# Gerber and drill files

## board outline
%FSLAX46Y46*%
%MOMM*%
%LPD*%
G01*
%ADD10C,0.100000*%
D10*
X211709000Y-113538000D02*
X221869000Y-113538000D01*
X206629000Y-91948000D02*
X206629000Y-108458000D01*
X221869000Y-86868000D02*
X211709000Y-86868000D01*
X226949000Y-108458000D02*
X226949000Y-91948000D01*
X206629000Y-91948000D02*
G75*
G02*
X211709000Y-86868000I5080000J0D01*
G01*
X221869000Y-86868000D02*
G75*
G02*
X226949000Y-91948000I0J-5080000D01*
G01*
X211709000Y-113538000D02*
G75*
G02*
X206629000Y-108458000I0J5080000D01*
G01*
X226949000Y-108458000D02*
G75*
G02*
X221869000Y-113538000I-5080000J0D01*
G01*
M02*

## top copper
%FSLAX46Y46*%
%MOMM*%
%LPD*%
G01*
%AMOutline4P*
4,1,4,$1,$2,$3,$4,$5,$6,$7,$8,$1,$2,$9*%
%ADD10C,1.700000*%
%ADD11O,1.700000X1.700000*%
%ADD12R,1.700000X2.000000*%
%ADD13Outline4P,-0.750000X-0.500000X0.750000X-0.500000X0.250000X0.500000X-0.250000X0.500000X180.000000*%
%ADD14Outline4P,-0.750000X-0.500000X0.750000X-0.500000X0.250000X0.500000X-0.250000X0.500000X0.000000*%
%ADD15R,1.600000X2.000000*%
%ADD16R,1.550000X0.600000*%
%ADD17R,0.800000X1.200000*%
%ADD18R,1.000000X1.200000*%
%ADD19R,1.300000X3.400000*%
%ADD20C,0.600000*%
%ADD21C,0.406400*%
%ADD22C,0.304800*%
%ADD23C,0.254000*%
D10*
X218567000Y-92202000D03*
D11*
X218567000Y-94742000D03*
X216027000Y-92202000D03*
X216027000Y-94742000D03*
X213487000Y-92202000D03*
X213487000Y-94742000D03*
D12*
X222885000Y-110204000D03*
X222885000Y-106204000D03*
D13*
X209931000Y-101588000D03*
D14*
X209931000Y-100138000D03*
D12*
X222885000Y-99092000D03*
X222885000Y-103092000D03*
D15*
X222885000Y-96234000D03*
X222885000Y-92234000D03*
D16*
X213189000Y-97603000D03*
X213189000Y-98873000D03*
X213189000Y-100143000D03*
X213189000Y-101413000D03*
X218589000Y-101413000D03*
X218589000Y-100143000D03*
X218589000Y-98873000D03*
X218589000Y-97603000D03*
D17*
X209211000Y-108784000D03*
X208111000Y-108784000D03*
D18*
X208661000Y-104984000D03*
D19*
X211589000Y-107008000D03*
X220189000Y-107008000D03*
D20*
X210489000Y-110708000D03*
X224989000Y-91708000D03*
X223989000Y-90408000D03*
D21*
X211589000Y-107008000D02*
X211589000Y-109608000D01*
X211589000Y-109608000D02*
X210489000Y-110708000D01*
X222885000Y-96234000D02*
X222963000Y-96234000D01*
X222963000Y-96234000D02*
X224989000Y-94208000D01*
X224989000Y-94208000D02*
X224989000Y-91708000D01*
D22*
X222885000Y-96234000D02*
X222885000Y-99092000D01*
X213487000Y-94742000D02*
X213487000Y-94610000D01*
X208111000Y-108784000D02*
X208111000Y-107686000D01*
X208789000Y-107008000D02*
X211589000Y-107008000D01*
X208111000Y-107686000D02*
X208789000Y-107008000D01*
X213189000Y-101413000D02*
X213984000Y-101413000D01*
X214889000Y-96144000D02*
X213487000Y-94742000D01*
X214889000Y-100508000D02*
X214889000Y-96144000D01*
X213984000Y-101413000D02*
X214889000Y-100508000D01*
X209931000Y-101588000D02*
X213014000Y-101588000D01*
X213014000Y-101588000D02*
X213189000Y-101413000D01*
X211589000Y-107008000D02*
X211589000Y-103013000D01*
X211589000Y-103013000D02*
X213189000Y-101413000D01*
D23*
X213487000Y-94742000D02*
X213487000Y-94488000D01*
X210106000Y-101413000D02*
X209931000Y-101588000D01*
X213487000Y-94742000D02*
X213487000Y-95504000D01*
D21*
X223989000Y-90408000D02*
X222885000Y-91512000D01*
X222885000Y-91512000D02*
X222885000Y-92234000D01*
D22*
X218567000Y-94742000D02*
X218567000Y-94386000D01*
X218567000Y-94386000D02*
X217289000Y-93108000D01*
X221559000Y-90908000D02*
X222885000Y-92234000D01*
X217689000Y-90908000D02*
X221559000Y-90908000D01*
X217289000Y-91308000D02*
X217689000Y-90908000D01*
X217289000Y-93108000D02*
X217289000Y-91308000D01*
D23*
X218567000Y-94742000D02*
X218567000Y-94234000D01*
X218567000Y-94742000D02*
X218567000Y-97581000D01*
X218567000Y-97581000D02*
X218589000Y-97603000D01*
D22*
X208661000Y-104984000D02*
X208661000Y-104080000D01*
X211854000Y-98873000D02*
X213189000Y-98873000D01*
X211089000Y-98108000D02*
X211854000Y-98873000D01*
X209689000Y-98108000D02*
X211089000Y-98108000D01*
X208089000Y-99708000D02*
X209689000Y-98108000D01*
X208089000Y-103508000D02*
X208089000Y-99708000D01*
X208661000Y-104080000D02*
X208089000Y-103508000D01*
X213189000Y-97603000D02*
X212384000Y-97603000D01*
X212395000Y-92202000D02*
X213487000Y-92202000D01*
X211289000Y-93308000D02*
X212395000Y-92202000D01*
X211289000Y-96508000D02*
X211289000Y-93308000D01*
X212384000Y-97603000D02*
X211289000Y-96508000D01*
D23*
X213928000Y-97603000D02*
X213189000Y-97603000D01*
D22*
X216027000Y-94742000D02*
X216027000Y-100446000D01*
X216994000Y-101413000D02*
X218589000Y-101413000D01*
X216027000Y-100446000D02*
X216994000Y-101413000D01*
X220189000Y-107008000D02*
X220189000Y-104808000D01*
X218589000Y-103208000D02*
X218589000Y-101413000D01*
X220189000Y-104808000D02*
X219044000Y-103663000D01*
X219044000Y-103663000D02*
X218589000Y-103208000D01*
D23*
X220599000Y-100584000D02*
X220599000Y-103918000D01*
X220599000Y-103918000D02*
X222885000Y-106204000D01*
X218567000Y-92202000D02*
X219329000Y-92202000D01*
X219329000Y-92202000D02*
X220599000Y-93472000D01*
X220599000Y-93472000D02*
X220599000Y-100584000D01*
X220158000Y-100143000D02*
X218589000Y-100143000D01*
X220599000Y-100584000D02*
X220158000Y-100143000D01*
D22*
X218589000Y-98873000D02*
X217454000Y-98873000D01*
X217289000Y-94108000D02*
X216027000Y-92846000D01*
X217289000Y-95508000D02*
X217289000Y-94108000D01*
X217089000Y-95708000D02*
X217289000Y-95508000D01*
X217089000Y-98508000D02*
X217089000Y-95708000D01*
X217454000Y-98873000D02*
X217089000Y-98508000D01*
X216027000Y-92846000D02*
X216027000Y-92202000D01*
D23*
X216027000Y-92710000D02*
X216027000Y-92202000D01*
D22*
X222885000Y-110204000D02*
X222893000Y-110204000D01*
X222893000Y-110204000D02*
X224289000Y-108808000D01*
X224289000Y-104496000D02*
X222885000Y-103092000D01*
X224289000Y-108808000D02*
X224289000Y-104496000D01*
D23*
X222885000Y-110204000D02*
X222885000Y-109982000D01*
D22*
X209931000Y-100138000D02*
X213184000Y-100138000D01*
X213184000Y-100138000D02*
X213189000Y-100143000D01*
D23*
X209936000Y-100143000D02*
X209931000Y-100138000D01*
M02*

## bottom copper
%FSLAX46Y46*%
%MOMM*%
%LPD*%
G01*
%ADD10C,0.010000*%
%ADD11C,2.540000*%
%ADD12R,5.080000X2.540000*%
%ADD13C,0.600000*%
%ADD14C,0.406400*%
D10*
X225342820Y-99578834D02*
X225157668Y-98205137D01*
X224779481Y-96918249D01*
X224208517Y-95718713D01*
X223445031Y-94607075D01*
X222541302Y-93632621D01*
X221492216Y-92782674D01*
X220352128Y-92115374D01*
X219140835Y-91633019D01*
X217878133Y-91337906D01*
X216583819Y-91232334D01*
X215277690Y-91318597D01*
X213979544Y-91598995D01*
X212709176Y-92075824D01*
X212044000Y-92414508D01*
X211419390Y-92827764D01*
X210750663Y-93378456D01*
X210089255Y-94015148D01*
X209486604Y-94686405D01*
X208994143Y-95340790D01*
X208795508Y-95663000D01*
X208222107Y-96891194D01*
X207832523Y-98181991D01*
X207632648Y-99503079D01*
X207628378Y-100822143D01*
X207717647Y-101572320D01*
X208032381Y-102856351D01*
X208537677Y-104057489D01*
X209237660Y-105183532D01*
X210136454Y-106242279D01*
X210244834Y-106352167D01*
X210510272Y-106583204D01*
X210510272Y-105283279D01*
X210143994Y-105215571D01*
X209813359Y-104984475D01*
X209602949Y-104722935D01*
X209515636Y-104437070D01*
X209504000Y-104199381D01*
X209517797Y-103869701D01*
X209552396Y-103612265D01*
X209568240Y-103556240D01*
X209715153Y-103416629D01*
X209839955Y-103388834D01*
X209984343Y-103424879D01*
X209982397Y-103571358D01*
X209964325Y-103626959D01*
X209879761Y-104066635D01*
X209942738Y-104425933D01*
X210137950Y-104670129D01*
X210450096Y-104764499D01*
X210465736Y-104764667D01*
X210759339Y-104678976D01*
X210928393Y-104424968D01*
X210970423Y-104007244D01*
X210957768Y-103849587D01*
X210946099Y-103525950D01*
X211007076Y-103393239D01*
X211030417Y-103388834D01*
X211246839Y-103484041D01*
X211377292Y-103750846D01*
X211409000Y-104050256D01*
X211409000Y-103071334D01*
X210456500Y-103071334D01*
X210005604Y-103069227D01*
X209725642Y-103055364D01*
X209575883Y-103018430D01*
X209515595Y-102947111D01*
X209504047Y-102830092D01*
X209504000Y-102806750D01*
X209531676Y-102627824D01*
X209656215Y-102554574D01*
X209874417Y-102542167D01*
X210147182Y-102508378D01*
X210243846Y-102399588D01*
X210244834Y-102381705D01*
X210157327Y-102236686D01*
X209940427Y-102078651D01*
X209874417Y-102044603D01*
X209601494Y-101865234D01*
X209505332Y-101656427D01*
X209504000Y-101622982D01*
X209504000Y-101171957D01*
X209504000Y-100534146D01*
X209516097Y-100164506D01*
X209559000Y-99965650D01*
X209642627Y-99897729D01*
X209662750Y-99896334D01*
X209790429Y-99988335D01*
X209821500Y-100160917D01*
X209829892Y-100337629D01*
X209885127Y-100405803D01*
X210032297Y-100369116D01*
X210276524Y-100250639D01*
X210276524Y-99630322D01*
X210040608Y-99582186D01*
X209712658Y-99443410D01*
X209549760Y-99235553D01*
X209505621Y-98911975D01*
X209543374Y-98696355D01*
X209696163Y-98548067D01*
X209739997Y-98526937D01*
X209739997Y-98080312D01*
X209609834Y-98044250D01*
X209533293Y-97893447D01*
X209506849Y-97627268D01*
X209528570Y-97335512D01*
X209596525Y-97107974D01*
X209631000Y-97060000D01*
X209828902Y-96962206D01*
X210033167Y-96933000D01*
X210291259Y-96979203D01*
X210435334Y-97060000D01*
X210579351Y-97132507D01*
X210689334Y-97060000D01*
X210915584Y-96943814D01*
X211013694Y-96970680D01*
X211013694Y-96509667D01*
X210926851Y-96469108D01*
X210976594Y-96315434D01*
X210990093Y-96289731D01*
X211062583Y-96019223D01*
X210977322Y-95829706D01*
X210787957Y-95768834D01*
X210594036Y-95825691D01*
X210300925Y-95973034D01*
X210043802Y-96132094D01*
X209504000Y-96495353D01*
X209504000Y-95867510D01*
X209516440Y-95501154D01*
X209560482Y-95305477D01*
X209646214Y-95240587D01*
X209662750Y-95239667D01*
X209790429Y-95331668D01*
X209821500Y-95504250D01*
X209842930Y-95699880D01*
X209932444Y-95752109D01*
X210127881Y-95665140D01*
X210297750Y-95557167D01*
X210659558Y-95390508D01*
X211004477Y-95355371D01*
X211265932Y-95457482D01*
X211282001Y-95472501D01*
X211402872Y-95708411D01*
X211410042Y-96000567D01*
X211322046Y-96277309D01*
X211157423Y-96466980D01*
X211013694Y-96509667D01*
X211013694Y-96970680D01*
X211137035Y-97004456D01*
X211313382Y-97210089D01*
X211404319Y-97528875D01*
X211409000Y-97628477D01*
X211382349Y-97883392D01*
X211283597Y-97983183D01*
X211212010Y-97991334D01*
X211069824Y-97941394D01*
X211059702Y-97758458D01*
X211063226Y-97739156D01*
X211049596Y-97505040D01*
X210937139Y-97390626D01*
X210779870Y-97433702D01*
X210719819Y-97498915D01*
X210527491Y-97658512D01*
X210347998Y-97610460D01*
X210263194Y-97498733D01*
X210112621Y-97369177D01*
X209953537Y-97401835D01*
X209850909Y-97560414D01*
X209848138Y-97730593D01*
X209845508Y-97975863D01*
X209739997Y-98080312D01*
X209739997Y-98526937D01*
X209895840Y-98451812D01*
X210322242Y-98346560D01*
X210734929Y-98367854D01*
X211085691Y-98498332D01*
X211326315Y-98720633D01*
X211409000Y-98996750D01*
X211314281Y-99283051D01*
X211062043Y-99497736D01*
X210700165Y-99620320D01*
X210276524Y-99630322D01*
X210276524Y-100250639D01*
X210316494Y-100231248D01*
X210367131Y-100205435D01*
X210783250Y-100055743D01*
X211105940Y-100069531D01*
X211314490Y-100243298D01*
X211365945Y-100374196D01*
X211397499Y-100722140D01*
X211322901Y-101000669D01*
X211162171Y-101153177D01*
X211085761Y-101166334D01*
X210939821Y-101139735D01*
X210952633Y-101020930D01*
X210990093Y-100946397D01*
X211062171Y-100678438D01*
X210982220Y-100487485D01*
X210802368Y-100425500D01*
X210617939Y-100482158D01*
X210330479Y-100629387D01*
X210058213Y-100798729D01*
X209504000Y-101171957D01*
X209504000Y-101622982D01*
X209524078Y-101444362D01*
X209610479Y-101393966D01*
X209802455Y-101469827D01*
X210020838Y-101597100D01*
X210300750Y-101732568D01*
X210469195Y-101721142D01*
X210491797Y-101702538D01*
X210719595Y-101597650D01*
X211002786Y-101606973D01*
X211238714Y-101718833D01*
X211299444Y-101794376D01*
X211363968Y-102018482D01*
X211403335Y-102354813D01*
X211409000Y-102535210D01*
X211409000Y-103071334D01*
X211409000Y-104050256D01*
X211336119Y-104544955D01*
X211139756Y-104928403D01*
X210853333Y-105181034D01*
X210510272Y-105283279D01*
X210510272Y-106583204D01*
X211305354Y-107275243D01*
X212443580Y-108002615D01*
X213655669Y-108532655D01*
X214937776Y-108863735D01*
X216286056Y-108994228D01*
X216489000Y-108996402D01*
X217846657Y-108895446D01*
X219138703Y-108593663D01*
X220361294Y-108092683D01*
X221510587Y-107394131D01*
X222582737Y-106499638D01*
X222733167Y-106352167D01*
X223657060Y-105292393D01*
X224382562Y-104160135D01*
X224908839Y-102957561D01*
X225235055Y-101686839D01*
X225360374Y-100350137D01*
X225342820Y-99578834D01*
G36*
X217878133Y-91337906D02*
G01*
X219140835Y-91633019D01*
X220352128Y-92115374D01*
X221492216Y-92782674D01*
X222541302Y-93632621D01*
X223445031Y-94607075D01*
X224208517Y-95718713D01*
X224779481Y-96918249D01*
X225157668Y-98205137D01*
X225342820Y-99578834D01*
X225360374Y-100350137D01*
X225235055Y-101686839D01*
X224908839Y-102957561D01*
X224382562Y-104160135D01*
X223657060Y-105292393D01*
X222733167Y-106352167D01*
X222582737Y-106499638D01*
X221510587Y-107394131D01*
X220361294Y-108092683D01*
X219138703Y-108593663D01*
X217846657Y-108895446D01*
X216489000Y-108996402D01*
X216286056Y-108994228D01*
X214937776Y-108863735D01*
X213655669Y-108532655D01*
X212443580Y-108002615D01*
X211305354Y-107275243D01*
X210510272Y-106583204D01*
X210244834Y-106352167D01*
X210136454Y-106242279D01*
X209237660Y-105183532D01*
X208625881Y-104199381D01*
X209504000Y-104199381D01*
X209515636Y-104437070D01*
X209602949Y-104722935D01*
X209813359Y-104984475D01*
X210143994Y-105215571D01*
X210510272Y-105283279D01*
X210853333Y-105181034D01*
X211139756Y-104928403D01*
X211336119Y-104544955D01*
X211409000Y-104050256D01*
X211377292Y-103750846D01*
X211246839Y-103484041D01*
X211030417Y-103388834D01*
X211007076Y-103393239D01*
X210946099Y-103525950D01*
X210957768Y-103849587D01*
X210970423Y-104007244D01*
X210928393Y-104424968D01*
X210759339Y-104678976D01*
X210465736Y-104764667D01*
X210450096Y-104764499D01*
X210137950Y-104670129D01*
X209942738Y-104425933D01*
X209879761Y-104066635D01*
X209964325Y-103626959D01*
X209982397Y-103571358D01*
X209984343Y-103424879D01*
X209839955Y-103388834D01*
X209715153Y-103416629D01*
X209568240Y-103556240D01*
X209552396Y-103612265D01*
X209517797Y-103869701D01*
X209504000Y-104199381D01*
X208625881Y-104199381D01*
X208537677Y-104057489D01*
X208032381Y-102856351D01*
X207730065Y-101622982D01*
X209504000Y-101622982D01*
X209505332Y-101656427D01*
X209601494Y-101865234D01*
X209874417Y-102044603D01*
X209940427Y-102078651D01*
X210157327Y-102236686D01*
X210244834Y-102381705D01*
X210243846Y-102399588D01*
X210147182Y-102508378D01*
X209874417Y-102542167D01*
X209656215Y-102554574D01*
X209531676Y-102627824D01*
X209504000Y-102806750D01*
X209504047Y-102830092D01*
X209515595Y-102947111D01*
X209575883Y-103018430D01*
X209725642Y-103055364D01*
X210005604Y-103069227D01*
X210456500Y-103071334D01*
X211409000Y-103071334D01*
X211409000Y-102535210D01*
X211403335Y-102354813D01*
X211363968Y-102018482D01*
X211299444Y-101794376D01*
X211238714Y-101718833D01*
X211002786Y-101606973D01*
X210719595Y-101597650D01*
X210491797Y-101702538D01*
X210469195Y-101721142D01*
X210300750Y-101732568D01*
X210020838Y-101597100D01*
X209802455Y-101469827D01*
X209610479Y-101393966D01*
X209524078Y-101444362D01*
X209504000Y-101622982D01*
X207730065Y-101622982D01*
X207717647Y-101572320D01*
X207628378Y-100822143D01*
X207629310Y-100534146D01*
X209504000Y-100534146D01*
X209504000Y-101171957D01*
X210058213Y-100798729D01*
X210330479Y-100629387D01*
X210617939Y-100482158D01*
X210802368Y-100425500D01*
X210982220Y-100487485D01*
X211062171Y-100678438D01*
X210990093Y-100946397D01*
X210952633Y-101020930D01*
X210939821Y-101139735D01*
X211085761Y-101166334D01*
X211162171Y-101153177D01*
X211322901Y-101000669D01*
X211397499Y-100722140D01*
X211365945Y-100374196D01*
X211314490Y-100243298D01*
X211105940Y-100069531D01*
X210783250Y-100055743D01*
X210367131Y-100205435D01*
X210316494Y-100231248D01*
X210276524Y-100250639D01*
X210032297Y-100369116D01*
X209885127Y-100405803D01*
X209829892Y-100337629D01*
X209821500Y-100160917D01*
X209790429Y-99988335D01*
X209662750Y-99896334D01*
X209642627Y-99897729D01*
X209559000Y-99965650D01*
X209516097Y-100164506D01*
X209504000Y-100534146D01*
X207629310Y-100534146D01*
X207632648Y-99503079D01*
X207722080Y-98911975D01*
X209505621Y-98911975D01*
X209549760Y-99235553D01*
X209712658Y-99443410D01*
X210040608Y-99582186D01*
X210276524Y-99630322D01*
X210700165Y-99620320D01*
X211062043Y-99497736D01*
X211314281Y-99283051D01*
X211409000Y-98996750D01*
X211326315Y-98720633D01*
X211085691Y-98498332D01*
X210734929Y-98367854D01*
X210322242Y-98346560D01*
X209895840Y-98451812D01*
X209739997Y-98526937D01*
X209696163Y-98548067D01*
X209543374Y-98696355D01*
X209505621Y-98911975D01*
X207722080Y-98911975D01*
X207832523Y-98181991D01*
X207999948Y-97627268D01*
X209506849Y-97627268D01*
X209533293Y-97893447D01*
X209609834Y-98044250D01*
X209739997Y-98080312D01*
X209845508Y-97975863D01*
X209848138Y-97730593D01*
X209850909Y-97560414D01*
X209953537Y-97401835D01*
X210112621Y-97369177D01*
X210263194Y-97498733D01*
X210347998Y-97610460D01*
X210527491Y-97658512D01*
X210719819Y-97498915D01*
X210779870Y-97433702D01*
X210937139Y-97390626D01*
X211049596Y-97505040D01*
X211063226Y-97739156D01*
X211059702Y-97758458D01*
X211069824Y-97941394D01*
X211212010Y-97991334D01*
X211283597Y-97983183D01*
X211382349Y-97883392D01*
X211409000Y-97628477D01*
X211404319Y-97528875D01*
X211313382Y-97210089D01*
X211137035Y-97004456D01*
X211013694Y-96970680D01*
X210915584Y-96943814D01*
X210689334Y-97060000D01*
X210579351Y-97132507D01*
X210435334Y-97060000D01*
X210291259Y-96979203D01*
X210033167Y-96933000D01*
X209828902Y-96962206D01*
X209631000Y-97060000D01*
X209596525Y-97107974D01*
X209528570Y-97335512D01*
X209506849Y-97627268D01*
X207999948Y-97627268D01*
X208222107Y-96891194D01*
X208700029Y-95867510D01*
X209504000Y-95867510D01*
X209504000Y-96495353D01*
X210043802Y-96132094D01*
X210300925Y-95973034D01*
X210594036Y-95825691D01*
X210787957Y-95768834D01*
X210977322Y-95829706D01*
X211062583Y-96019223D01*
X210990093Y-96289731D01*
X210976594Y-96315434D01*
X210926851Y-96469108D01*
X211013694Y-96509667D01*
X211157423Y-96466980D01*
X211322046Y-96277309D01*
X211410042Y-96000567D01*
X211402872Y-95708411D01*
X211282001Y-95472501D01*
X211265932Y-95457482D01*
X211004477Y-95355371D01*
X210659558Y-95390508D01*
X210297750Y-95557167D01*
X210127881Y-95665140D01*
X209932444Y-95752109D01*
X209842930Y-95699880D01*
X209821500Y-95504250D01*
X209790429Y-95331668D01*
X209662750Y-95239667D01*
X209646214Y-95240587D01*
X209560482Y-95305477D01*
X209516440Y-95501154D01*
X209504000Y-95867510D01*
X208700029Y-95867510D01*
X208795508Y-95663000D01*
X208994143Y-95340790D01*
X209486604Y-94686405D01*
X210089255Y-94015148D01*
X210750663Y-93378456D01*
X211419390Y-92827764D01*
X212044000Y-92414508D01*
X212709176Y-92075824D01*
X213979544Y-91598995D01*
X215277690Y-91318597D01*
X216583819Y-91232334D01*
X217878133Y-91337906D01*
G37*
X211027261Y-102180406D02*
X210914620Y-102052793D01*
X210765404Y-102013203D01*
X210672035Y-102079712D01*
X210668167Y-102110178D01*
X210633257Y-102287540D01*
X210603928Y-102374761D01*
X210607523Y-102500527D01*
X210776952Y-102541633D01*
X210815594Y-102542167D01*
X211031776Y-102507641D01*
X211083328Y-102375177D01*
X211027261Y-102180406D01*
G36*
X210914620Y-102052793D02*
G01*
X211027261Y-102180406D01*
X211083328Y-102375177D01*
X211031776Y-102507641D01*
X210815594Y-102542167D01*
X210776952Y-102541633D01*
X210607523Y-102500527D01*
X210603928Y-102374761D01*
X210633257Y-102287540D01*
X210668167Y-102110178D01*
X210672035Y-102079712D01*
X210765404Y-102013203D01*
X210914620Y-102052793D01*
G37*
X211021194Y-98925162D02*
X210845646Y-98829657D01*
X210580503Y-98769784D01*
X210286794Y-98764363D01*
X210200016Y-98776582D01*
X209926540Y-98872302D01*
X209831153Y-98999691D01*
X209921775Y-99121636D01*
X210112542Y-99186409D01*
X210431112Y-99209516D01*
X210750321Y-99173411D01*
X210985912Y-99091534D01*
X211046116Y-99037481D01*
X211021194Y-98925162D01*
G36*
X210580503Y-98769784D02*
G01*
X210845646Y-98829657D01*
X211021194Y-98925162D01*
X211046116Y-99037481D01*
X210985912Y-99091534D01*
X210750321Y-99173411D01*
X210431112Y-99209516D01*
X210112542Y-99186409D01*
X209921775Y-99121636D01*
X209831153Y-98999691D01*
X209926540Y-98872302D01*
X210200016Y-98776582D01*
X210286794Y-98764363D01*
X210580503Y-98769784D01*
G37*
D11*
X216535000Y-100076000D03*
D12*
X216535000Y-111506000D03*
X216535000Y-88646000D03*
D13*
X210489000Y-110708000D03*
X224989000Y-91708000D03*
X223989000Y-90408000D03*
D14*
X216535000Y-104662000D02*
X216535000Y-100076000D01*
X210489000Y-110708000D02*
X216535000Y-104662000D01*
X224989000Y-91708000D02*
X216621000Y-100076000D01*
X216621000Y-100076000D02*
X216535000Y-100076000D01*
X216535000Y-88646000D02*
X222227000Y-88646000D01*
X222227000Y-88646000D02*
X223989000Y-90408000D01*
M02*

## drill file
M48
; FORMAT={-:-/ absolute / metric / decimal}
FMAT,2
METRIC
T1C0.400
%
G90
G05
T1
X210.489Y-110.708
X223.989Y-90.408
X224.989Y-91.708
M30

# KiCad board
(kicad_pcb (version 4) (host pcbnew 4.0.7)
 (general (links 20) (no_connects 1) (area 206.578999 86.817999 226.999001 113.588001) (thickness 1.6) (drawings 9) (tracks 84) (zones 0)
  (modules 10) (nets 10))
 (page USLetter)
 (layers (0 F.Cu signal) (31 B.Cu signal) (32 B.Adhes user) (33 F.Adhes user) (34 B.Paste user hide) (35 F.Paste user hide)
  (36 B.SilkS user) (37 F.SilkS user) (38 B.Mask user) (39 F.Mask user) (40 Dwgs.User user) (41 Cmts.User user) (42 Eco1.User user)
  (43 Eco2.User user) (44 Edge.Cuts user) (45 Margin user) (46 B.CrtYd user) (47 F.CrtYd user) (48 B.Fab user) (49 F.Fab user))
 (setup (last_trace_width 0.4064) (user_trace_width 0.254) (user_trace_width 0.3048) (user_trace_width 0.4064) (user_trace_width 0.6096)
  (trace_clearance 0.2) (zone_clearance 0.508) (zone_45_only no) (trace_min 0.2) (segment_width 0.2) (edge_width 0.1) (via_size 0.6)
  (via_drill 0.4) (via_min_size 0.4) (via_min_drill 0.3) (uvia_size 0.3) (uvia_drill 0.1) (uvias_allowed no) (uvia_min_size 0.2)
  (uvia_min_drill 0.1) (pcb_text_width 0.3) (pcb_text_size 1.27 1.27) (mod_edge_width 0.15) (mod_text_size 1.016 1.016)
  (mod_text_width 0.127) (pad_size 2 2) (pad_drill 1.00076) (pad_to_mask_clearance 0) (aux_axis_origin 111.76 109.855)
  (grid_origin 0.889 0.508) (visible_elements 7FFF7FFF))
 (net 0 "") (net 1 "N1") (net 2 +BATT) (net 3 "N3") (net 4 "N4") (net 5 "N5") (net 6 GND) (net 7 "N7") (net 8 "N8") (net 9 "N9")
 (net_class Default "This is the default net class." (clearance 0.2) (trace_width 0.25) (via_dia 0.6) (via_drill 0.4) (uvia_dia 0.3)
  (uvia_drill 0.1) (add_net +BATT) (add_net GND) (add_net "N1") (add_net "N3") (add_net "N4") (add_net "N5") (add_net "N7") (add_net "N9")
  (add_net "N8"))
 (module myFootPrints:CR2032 (layer B.Cu) (at 216.489 100.108 90)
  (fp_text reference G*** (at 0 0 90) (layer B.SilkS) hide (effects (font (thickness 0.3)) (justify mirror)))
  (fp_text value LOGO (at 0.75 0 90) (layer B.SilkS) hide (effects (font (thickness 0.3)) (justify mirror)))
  (fp_poly
   (pts (xy 0.529166 8.85382) (xy 1.902863 8.668668) (xy 3.189751 8.290481) (xy 4.389287 7.719517) (xy 5.500925 6.956031)
    (xy 6.475379 6.052302) (xy 7.325326 5.003216) (xy 7.992626 3.863128) (xy 8.474981 2.651835) (xy 8.770094 1.389133)
    (xy 8.875666 0.094819) (xy 8.789403 -1.21131) (xy 8.509005 -2.509456) (xy 8.032176 -3.779824) (xy 7.693492 -4.445)
    (xy 7.280236 -5.06961) (xy 6.729544 -5.738337) (xy 6.092852 -6.399745) (xy 5.421595 -7.002396) (xy 4.76721 -7.494857)
    (xy 4.445 -7.693492) (xy 3.216806 -8.266893) (xy 1.926009 -8.656477) (xy 0.604921 -8.856352) (xy -0.714143 -8.860622)
    (xy -1.46432 -8.771353) (xy -2.748351 -8.456619) (xy -3.949489 -7.951323) (xy -5.075532 -7.25134) (xy -6.134279 -6.352546)
    (xy -6.244167 -6.244166) (xy -6.475204 -5.978728) (xy -5.175279 -5.978728) (xy -5.107571 -6.345006) (xy -4.876475 -6.675641)
    (xy -4.614935 -6.886051) (xy -4.32907 -6.973364) (xy -4.091381 -6.985) (xy -3.761701 -6.971203) (xy -3.504265 -6.936604)
    (xy -3.44824 -6.92076) (xy -3.308629 -6.773847) (xy -3.280834 -6.649045) (xy -3.316879 -6.504657) (xy -3.463358 -6.506603)
    (xy -3.518959 -6.524675) (xy -3.958635 -6.609239) (xy -4.317933 -6.546262) (xy -4.562129 -6.35105) (xy -4.656499 -6.038904)
    (xy -4.656667 -6.023264) (xy -4.570976 -5.729661) (xy -4.316968 -5.560607) (xy -3.899244 -5.518577) (xy -3.741587 -5.531232)
    (xy -3.41795 -5.542901) (xy -3.285239 -5.481924) (xy -3.280834 -5.458583) (xy -3.376041 -5.242161) (xy -3.642846 -5.111708)
    (xy -3.942256 -5.08) (xy -2.963334 -5.08) (xy -2.963334 -6.0325) (xy -2.961227 -6.483396) (xy -2.947364 -6.763358)
    (xy -2.91043 -6.913117) (xy -2.839111 -6.973405) (xy -2.722092 -6.984953) (xy -2.69875 -6.985) (xy -2.519824 -6.957324)
    (xy -2.446574 -6.832785) (xy -2.434167 -6.614583) (xy -2.400378 -6.341818) (xy -2.291588 -6.245154) (xy -2.273705 -6.244166)
    (xy -2.128686 -6.331673) (xy -1.970651 -6.548573) (xy -1.936603 -6.614583) (xy -1.757234 -6.887506) (xy -1.548427 -6.983668)
    (xy -1.514982 -6.985) (xy -1.063957 -6.985) (xy -0.426146 -6.985) (xy -0.056506 -6.972903) (xy 0.14235 -6.93) (xy 0.210271 -6.846373)
    (xy 0.211666 -6.82625) (xy 0.119665 -6.698571) (xy -0.052917 -6.6675) (xy -0.229629 -6.659108) (xy -0.297803 -6.603873)
    (xy -0.261116 -6.456703) (xy -0.142639 -6.212476) (xy 0.477678 -6.212476) (xy 0.525814 -6.448392) (xy 0.66459 -6.776342)
    (xy 0.872447 -6.93924) (xy 1.196025 -6.983379) (xy 1.411645 -6.945626) (xy 1.559933 -6.792837) (xy 1.581063 -6.749003)
    (xy 2.027688 -6.749003) (xy 2.06375 -6.879166) (xy 2.214553 -6.955707) (xy 2.480732 -6.982151) (xy 2.772488 -6.96043)
    (xy 3.000026 -6.892475) (xy 3.048 -6.858) (xy 3.145794 -6.660098) (xy 3.175 -6.455833) (xy 3.128797 -6.197741) (xy 3.048 -6.053666)
    (xy 2.975493 -5.909649) (xy 3.048 -5.799666) (xy 3.164186 -5.573416) (xy 3.13732 -5.475306) (xy 3.598333 -5.475306)
    (xy 3.638892 -5.562149) (xy 3.792566 -5.512406) (xy 3.818269 -5.498907) (xy 4.088777 -5.426417) (xy 4.278294 -5.511678)
    (xy 4.339166 -5.701043) (xy 4.282309 -5.894964) (xy 4.134966 -6.188075) (xy 3.975906 -6.445198) (xy 3.612647 -6.985) (xy 4.24049 -6.985)
    (xy 4.606846 -6.97256) (xy 4.802523 -6.928518) (xy 4.867413 -6.842786) (xy 4.868333 -6.82625) (xy 4.776332 -6.698571)
    (xy 4.60375 -6.6675) (xy 4.40812 -6.64607) (xy 4.355891 -6.556556) (xy 4.44286 -6.361119) (xy 4.550833 -6.19125) (xy 4.717492 -5.829442)
    (xy 4.752629 -5.484523) (xy 4.650518 -5.223068) (xy 4.635499 -5.206999) (xy 4.399589 -5.086128) (xy 4.107433 -5.078958)
    (xy 3.830691 -5.166954) (xy 3.64102 -5.331577) (xy 3.598333 -5.475306) (xy 3.13732 -5.475306) (xy 3.103544 -5.351965)
    (xy 2.897911 -5.175618) (xy 2.579125 -5.084681) (xy 2.479523 -5.08) (xy 2.224608 -5.106651) (xy 2.124817 -5.205403)
    (xy 2.116666 -5.27699) (xy 2.166606 -5.419176) (xy 2.349542 -5.429298) (xy 2.368844 -5.425774) (xy 2.60296 -5.439404)
    (xy 2.717374 -5.551861) (xy 2.674298 -5.70913) (xy 2.609085 -5.769181) (xy 2.449488 -5.961509) (xy 2.49754 -6.141002)
    (xy 2.609267 -6.225806) (xy 2.738823 -6.376379) (xy 2.706165 -6.535463) (xy 2.547586 -6.638091) (xy 2.377407 -6.640862)
    (xy 2.132137 -6.643492) (xy 2.027688 -6.749003) (xy 1.581063 -6.749003) (xy 1.656188 -6.59316) (xy 1.76144 -6.166758)
    (xy 1.740146 -5.754071) (xy 1.609668 -5.403309) (xy 1.387367 -5.162685) (xy 1.11125 -5.08) (xy 0.824949 -5.174719)
    (xy 0.610264 -5.426957) (xy 0.48768 -5.788835) (xy 0.477678 -6.212476) (xy -0.142639 -6.212476) (xy -0.123248 -6.172506)
    (xy -0.097435 -6.121869) (xy 0.052257 -5.70575) (xy 0.038469 -5.38306) (xy -0.135298 -5.17451) (xy -0.266196 -5.123055)
    (xy -0.61414 -5.091501) (xy -0.892669 -5.166099) (xy -1.045177 -5.326829) (xy -1.058334 -5.403239) (xy -1.031735 -5.549179)
    (xy -0.91293 -5.536367) (xy -0.838397 -5.498907) (xy -0.570438 -5.426829) (xy -0.379485 -5.50678) (xy -0.3175 -5.686632)
    (xy -0.374158 -5.871061) (xy -0.521387 -6.158521) (xy -0.690729 -6.430787) (xy -1.063957 -6.985) (xy -1.514982 -6.985)
    (xy -1.336362 -6.964922) (xy -1.285966 -6.878521) (xy -1.361827 -6.686545) (xy -1.4891 -6.468162) (xy -1.624568 -6.18825)
    (xy -1.613142 -6.019805) (xy -1.594538 -5.997203) (xy -1.48965 -5.769405) (xy -1.498973 -5.486214) (xy -1.610833 -5.250286)
    (xy -1.686376 -5.189556) (xy -1.910482 -5.125032) (xy -2.246813 -5.085665) (xy -2.42721 -5.08) (xy -2.963334 -5.08) (xy -3.942256 -5.08)
    (xy -4.436955 -5.152881) (xy -4.820403 -5.349244) (xy -5.073034 -5.635667) (xy -5.175279 -5.978728) (xy -6.475204 -5.978728)
    (xy -7.167243 -5.183646) (xy -7.894615 -4.04542) (xy -8.424655 -2.833331) (xy -8.755735 -1.551224) (xy -8.886228 -0.202944)
    (xy -8.888402 0) (xy -8.787446 1.357657) (xy -8.485663 2.649703) (xy -7.984683 3.872294) (xy -7.286131 5.021587) (xy -6.391638 6.093737)
    (xy -6.244167 6.244167) (xy -5.184393 7.16806) (xy -4.052135 7.893562) (xy -2.849561 8.419839) (xy -1.578839 8.746055)
    (xy -0.242137 8.871374) (xy 0.529166 8.85382))
   (layer B.Cu) (width 0.01))
  (fp_poly
   (pts (xy -2.072406 -5.461739) (xy -1.944793 -5.57438) (xy -1.905203 -5.723596) (xy -1.971712 -5.816965) (xy -2.002178 -5.820833)
    (xy -2.17954 -5.855743) (xy -2.266761 -5.885072) (xy -2.392527 -5.881477) (xy -2.433633 -5.712048) (xy -2.434167 -5.673406)
    (xy -2.399641 -5.457224) (xy -2.267177 -5.405672) (xy -2.072406 -5.461739))
   (layer B.Cu) (width 0.01))
  (fp_poly
   (pts (xy 1.182838 -5.467806) (xy 1.278343 -5.643354) (xy 1.338216 -5.908497) (xy 1.343637 -6.202206) (xy 1.331418 -6.288984)
    (xy 1.235698 -6.56246) (xy 1.108309 -6.657847) (xy 0.986364 -6.567225) (xy 0.921591 -6.376458) (xy 0.898484 -6.057888)
    (xy 0.934589 -5.738679) (xy 1.016466 -5.503088) (xy 1.070519 -5.442884) (xy 1.182838 -5.467806))
   (layer B.Cu) (width 0.01))
  (pad 3 smd circle (at 0 0 90) (size 17.78 17.78) (layers B.Paste B.Mask)))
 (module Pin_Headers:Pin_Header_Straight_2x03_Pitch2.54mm (layer F.Cu) (at 218.567 92.202 270)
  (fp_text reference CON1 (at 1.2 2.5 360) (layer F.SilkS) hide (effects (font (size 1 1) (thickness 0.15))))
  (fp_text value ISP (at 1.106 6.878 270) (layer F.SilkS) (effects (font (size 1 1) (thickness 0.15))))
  (pad 1 smd circle (at 0 0 270) (size 1.7 1.7) (layers F.Cu F.Paste F.Mask) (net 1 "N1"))
  (pad 2 smd oval (at 2.54 0 270) (size 1.7 1.7) (layers F.Cu F.Paste F.Mask) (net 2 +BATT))
  (pad 3 smd oval (at 0 2.54 270) (size 1.7 1.7) (layers F.Cu F.Paste F.Mask) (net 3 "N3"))
  (pad 4 smd oval (at 2.54 2.54 270) (size 1.7 1.7) (layers F.Cu F.Paste F.Mask) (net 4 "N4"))
  (pad 5 smd oval (at 0 5.08 270) (size 1.7 1.7) (layers F.Cu F.Paste F.Mask) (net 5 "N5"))
  (pad 6 smd oval (at 2.54 5.08 270) (size 1.7 1.7) (layers F.Cu F.Paste F.Mask) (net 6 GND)))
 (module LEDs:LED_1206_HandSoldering (layer F.Cu) (at 222.885 108.204 90)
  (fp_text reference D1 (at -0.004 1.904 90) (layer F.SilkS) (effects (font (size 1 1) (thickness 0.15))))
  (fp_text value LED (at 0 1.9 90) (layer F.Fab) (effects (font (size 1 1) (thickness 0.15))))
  (pad 1 smd rect (at -2 0 90) (size 2 1.7) (layers F.Cu F.Paste F.Mask) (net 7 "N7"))
  (pad 2 smd rect (at 2 0 90) (size 2 1.7) (layers F.Cu F.Paste F.Mask) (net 1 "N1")))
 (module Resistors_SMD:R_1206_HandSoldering (layer F.Cu) (at 209.931 100.838 90)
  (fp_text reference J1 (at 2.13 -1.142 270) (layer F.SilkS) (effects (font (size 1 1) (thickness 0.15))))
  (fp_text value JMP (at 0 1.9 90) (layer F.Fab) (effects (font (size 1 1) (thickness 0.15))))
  (pad 1 smd trapezoid (at -0.75 0 180) (size 1 1) (rect_delta 0 0.5) (layers F.Cu F.Paste F.Mask) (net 6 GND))
  (pad 2 smd trapezoid (at 0.7 0) (size 1 1) (rect_delta 0 0.5) (layers F.Cu F.Paste F.Mask) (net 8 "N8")))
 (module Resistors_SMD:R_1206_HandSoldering (layer F.Cu) (at 222.885 101.092 270)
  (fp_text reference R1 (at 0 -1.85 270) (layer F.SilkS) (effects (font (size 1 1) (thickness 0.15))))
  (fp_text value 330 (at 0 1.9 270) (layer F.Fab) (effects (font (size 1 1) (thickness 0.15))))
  (pad 1 smd rect (at -2 0 270) (size 2 1.7) (layers F.Cu F.Paste F.Mask) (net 6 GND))
  (pad 2 smd rect (at 2 0 270) (size 2 1.7) (layers F.Cu F.Paste F.Mask) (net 7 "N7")))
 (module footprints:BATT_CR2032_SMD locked (layer B.Cu) (at 216.535 100.076 90)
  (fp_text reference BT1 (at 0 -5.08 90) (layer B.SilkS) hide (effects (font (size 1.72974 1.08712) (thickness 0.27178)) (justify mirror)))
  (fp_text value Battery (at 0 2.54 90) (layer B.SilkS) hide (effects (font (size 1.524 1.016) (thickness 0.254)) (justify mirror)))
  (pad 2 smd circle (at 0 0 90) (size 2.54 2.54) (layers B.Cu B.Paste B.Mask) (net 6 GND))
  (pad 1 smd rect (at -11.43 0 90) (size 2.54 5.08) (layers B.Cu B.Paste B.Mask) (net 2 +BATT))
  (pad 1 smd rect (at 11.43 0 90) (size 2.54 5.08) (layers B.Cu B.Paste B.Mask) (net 2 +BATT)))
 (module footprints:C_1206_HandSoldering (layer F.Cu) (at 222.885 94.234 90)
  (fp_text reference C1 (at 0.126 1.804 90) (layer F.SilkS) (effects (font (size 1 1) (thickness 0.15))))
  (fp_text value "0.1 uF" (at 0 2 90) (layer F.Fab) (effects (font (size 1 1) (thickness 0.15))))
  (pad 1 smd rect (at -2 0 90) (size 2 1.6) (layers F.Cu F.Paste F.Mask) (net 6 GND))
  (pad 2 smd rect (at 2 0 90) (size 2 1.6) (layers F.Cu F.Paste F.Mask) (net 2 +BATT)))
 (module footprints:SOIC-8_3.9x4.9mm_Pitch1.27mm (layer F.Cu) (at 215.889 99.508)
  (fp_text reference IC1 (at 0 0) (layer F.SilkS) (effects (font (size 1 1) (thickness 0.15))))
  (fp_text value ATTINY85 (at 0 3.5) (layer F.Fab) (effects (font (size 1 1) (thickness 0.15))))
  (pad 1 smd rect (at -2.7 -1.905) (size 1.55 0.6) (layers F.Cu F.Paste F.Mask) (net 5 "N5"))
  (pad 2 smd rect (at -2.7 -0.635) (size 1.55 0.6) (layers F.Cu F.Paste F.Mask) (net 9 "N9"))
  (pad 3 smd rect (at -2.7 0.635) (size 1.55 0.6) (layers F.Cu F.Paste F.Mask) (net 8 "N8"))
  (pad 4 smd rect (at -2.7 1.905) (size 1.55 0.6) (layers F.Cu F.Paste F.Mask) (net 6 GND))
  (pad 5 smd rect (at 2.7 1.905) (size 1.55 0.6) (layers F.Cu F.Paste F.Mask) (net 4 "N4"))
  (pad 6 smd rect (at 2.7 0.635) (size 1.55 0.6) (layers F.Cu F.Paste F.Mask) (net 1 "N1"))
  (pad 7 smd rect (at 2.7 -0.635) (size 1.55 0.6) (layers F.Cu F.Paste F.Mask) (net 3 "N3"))
  (pad 8 smd rect (at 2.7 -1.905) (size 1.55 0.6) (layers F.Cu F.Paste F.Mask) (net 2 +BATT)))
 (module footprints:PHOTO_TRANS (layer F.Cu) (at 208.661 106.934 90)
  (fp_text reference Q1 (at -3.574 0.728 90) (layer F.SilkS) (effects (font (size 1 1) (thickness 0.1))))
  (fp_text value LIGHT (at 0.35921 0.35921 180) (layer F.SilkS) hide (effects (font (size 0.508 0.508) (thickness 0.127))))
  (pad 2 smd rect (at -1.85 0.55 90) (size 1.2 0.8) (layers F.Cu F.Paste F.Mask))
  (pad 1 smd rect (at -1.85 -0.55 90) (size 1.2 0.8) (layers F.Cu F.Paste F.Mask) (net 6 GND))
  (pad 3 connect rect (at 1.95 0 90) (size 1.2 1) (layers F.Cu F.Mask) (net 9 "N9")))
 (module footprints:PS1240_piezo (layer F.Cu) (at 215.889 107.008)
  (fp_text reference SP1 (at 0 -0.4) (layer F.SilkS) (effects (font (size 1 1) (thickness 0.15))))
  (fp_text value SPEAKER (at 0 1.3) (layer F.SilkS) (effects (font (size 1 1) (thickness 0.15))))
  (pad 1 smd rect (at -4.3 0) (size 1.3 3.4) (layers F.Cu F.Paste F.Mask) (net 6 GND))
  (pad 2 smd rect (at 4.3 0) (size 1.3 3.4) (layers F.Cu F.Paste F.Mask) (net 4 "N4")))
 (gr_line (start 211.709 113.538) (end 221.869 113.538) (angle 90) (layer Edge.Cuts) (width 0.1))
 (gr_line (start 206.629 91.948) (end 206.629 108.458) (angle 90) (layer Edge.Cuts) (width 0.1))
 (gr_line (start 221.869 86.868) (end 211.709 86.868) (angle 90) (layer Edge.Cuts) (width 0.1))
 (gr_line (start 226.949 108.458) (end 226.949 91.948) (angle 90) (layer Edge.Cuts) (width 0.1))
 (gr_arc (start 211.709 91.948) (end 206.629 91.948) (angle 90) (layer Edge.Cuts) (width 0.1))
 (gr_arc (start 221.869 91.948) (end 221.869 86.868) (angle 90) (layer Edge.Cuts) (width 0.1))
 (gr_arc (start 211.709 108.458) (end 211.709 113.538) (angle 90) (layer Edge.Cuts) (width 0.1))
 (gr_arc (start 221.869 108.458) (end 226.949 108.458) (angle 90) (layer Edge.Cuts) (width 0.1))
 (segment (start 211.589 107.008) (end 211.589 109.608) (width 0.4064) (layer F.Cu) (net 6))
 (segment (start 216.535 104.662) (end 216.535 100.076) (width 0.4064) (layer B.Cu) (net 6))
 (segment (start 210.489 110.708) (end 216.535 104.662) (width 0.4064) (layer B.Cu) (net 6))
 (via (at 210.489 110.708) (size 0.6) (drill 0.4) (layers F.Cu B.Cu) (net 6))
 (segment (start 211.589 109.608) (end 210.489 110.708) (width 0.4064) (layer F.Cu) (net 6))
 (segment (start 222.885 96.234) (end 222.963 96.234) (width 0.4064) (layer F.Cu) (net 6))
 (segment (start 222.963 96.234) (end 224.989 94.208) (width 0.4064) (layer F.Cu) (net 6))
 (segment (start 224.989 91.708) (end 216.621 100.076) (width 0.4064) (layer B.Cu) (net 6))
 (via (at 224.989 91.708) (size 0.6) (drill 0.4) (layers F.Cu B.Cu) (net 6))
 (segment (start 224.989 94.208) (end 224.989 91.708) (width 0.4064) (layer F.Cu) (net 6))
 (segment (start 216.621 100.076) (end 216.535 100.076) (width 0.4064) (layer B.Cu) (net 6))
 (segment (start 222.885 96.234) (end 222.885 99.092) (width 0.3048) (layer F.Cu) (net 6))
 (segment (start 213.487 94.742) (end 213.487 94.61) (width 0.3048) (layer F.Cu) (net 6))
 (segment (start 208.111 108.784) (end 208.111 107.686) (width 0.3048) (layer F.Cu) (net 6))
 (segment (start 208.789 107.008) (end 211.589 107.008) (width 0.3048) (layer F.Cu) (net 6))
 (segment (start 208.111 107.686) (end 208.789 107.008) (width 0.3048) (layer F.Cu) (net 6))
 (segment (start 213.189 101.413) (end 213.984 101.413) (width 0.3048) (layer F.Cu) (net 6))
 (segment (start 214.889 96.144) (end 213.487 94.742) (width 0.3048) (layer F.Cu) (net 6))
 (segment (start 214.889 100.508) (end 214.889 96.144) (width 0.3048) (layer F.Cu) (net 6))
 (segment (start 213.984 101.413) (end 214.889 100.508) (width 0.3048) (layer F.Cu) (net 6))
 (segment (start 209.931 101.588) (end 213.014 101.588) (width 0.3048) (layer F.Cu) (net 6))
 (segment (start 213.014 101.588) (end 213.189 101.413) (width 0.3048) (layer F.Cu) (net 6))
 (segment (start 211.589 107.008) (end 211.589 103.013) (width 0.3048) (layer F.Cu) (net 6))
 (segment (start 211.589 103.013) (end 213.189 101.413) (width 0.3048) (layer F.Cu) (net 6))
 (segment (start 213.487 94.742) (end 213.487 94.488) (width 0.254) (layer F.Cu) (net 6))
 (segment (start 210.106 101.413) (end 209.931 101.588) (width 0.254) (layer F.Cu) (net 6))
 (segment (start 213.487 94.742) (end 213.487 95.504) (width 0.254) (layer F.Cu) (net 6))
 (segment (start 216.535 88.646) (end 222.227 88.646) (width 0.4064) (layer B.Cu) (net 2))
 (segment (start 223.989 90.408) (end 222.885 91.512) (width 0.4064) (layer F.Cu) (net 2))
 (via (at 223.989 90.408) (size 0.6) (drill 0.4) (layers F.Cu B.Cu) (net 2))
 (segment (start 222.227 88.646) (end 223.989 90.408) (width 0.4064) (layer B.Cu) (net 2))
 (segment (start 222.885 91.512) (end 222.885 92.234) (width 0.4064) (layer F.Cu) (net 2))
 (segment (start 218.567 94.742) (end 218.567 94.386) (width 0.3048) (layer F.Cu) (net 2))
 (segment (start 218.567 94.386) (end 217.289 93.108) (width 0.3048) (layer F.Cu) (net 2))
 (segment (start 221.559 90.908) (end 222.885 92.234) (width 0.3048) (layer F.Cu) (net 2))
 (segment (start 217.689 90.908) (end 221.559 90.908) (width 0.3048) (layer F.Cu) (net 2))
 (segment (start 217.289 91.308) (end 217.689 90.908) (width 0.3048) (layer F.Cu) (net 2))
 (segment (start 217.289 93.108) (end 217.289 91.308) (width 0.3048) (layer F.Cu) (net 2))
 (segment (start 218.567 94.742) (end 218.567 94.234) (width 0.254) (layer F.Cu) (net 2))
 (segment (start 218.567 94.742) (end 218.567 97.581) (width 0.254) (layer F.Cu) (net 2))
 (segment (start 218.567 97.581) (end 218.589 97.603) (width 0.254) (layer F.Cu) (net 2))
 (segment (start 208.661 104.984) (end 208.661 104.08) (width 0.3048) (layer F.Cu) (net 9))
 (segment (start 211.854 98.873) (end 213.189 98.873) (width 0.3048) (layer F.Cu) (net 9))
 (segment (start 211.089 98.108) (end 211.854 98.873) (width 0.3048) (layer F.Cu) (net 9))
 (segment (start 209.689 98.108) (end 211.089 98.108) (width 0.3048) (layer F.Cu) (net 9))
 (segment (start 208.089 99.708) (end 209.689 98.108) (width 0.3048) (layer F.Cu) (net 9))
 (segment (start 208.089 103.508) (end 208.089 99.708) (width 0.3048) (layer F.Cu) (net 9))
 (segment (start 208.661 104.08) (end 208.089 103.508) (width 0.3048) (layer F.Cu) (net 9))
 (segment (start 213.189 97.603) (end 212.384 97.603) (width 0.3048) (layer F.Cu) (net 5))
 (segment (start 212.395 92.202) (end 213.487 92.202) (width 0.3048) (layer F.Cu) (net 5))
 (segment (start 211.289 93.308) (end 212.395 92.202) (width 0.3048) (layer F.Cu) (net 5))
 (segment (start 211.289 96.508) (end 211.289 93.308) (width 0.3048) (layer F.Cu) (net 5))
 (segment (start 212.384 97.603) (end 211.289 96.508) (width 0.3048) (layer F.Cu) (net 5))
 (segment (start 213.928 97.603) (end 213.189 97.603) (width 0.254) (layer F.Cu) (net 5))
 (segment (start 216.027 94.742) (end 216.027 100.446) (width 0.3048) (layer F.Cu) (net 4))
 (segment (start 216.994 101.413) (end 218.589 101.413) (width 0.3048) (layer F.Cu) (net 4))
 (segment (start 216.027 100.446) (end 216.994 101.413) (width 0.3048) (layer F.Cu) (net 4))
 (segment (start 220.189 107.008) (end 220.189 104.808) (width 0.3048) (layer F.Cu) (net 4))
 (segment (start 218.589 103.208) (end 218.589 101.413) (width 0.3048) (layer F.Cu) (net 4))
 (segment (start 220.189 104.808) (end 219.044 103.663) (width 0.3048) (layer F.Cu) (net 4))
 (segment (start 219.044 103.663) (end 218.589 103.208) (width 0.3048) (layer F.Cu) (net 4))
 (segment (start 220.599 100.584) (end 220.599 103.918) (width 0.254) (layer F.Cu) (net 1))
 (segment (start 220.599 103.918) (end 222.885 106.204) (width 0.254) (layer F.Cu) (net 1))
 (segment (start 218.567 92.202) (end 219.329 92.202) (width 0.254) (layer F.Cu) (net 1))
 (segment (start 219.329 92.202) (end 220.599 93.472) (width 0.254) (layer F.Cu) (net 1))
 (segment (start 220.599 93.472) (end 220.599 100.584) (width 0.254) (layer F.Cu) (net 1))
 (segment (start 220.158 100.143) (end 218.589 100.143) (width 0.254) (layer F.Cu) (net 1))
 (segment (start 220.599 100.584) (end 220.158 100.143) (width 0.254) (layer F.Cu) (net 1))
 (segment (start 218.589 98.873) (end 217.454 98.873) (width 0.3048) (layer F.Cu) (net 3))
 (segment (start 217.289 94.108) (end 216.027 92.846) (width 0.3048) (layer F.Cu) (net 3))
 (segment (start 217.289 95.508) (end 217.289 94.108) (width 0.3048) (layer F.Cu) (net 3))
 (segment (start 217.089 95.708) (end 217.289 95.508) (width 0.3048) (layer F.Cu) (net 3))
 (segment (start 217.089 98.508) (end 217.089 95.708) (width 0.3048) (layer F.Cu) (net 3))
 (segment (start 217.454 98.873) (end 217.089 98.508) (width 0.3048) (layer F.Cu) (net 3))
 (segment (start 216.027 92.846) (end 216.027 92.202) (width 0.3048) (layer F.Cu) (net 3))
 (segment (start 216.027 92.71) (end 216.027 92.202) (width 0.254) (layer F.Cu) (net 3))
 (segment (start 222.885 110.204) (end 222.893 110.204) (width 0.3048) (layer F.Cu) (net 7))
 (segment (start 222.893 110.204) (end 224.289 108.808) (width 0.3048) (layer F.Cu) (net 7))
 (segment (start 224.289 104.496) (end 222.885 103.092) (width 0.3048) (layer F.Cu) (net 7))
 (segment (start 224.289 108.808) (end 224.289 104.496) (width 0.3048) (layer F.Cu) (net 7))
 (segment (start 222.885 110.204) (end 222.885 109.982) (width 0.254) (layer F.Cu) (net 7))
 (segment (start 209.931 100.138) (end 213.184 100.138) (width 0.3048) (layer F.Cu) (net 8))
 (segment (start 213.184 100.138) (end 213.189 100.143) (width 0.3048) (layer F.Cu) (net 8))
 (segment (start 209.936 100.143) (end 209.931 100.138) (width 0.254) (layer F.Cu) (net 8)))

